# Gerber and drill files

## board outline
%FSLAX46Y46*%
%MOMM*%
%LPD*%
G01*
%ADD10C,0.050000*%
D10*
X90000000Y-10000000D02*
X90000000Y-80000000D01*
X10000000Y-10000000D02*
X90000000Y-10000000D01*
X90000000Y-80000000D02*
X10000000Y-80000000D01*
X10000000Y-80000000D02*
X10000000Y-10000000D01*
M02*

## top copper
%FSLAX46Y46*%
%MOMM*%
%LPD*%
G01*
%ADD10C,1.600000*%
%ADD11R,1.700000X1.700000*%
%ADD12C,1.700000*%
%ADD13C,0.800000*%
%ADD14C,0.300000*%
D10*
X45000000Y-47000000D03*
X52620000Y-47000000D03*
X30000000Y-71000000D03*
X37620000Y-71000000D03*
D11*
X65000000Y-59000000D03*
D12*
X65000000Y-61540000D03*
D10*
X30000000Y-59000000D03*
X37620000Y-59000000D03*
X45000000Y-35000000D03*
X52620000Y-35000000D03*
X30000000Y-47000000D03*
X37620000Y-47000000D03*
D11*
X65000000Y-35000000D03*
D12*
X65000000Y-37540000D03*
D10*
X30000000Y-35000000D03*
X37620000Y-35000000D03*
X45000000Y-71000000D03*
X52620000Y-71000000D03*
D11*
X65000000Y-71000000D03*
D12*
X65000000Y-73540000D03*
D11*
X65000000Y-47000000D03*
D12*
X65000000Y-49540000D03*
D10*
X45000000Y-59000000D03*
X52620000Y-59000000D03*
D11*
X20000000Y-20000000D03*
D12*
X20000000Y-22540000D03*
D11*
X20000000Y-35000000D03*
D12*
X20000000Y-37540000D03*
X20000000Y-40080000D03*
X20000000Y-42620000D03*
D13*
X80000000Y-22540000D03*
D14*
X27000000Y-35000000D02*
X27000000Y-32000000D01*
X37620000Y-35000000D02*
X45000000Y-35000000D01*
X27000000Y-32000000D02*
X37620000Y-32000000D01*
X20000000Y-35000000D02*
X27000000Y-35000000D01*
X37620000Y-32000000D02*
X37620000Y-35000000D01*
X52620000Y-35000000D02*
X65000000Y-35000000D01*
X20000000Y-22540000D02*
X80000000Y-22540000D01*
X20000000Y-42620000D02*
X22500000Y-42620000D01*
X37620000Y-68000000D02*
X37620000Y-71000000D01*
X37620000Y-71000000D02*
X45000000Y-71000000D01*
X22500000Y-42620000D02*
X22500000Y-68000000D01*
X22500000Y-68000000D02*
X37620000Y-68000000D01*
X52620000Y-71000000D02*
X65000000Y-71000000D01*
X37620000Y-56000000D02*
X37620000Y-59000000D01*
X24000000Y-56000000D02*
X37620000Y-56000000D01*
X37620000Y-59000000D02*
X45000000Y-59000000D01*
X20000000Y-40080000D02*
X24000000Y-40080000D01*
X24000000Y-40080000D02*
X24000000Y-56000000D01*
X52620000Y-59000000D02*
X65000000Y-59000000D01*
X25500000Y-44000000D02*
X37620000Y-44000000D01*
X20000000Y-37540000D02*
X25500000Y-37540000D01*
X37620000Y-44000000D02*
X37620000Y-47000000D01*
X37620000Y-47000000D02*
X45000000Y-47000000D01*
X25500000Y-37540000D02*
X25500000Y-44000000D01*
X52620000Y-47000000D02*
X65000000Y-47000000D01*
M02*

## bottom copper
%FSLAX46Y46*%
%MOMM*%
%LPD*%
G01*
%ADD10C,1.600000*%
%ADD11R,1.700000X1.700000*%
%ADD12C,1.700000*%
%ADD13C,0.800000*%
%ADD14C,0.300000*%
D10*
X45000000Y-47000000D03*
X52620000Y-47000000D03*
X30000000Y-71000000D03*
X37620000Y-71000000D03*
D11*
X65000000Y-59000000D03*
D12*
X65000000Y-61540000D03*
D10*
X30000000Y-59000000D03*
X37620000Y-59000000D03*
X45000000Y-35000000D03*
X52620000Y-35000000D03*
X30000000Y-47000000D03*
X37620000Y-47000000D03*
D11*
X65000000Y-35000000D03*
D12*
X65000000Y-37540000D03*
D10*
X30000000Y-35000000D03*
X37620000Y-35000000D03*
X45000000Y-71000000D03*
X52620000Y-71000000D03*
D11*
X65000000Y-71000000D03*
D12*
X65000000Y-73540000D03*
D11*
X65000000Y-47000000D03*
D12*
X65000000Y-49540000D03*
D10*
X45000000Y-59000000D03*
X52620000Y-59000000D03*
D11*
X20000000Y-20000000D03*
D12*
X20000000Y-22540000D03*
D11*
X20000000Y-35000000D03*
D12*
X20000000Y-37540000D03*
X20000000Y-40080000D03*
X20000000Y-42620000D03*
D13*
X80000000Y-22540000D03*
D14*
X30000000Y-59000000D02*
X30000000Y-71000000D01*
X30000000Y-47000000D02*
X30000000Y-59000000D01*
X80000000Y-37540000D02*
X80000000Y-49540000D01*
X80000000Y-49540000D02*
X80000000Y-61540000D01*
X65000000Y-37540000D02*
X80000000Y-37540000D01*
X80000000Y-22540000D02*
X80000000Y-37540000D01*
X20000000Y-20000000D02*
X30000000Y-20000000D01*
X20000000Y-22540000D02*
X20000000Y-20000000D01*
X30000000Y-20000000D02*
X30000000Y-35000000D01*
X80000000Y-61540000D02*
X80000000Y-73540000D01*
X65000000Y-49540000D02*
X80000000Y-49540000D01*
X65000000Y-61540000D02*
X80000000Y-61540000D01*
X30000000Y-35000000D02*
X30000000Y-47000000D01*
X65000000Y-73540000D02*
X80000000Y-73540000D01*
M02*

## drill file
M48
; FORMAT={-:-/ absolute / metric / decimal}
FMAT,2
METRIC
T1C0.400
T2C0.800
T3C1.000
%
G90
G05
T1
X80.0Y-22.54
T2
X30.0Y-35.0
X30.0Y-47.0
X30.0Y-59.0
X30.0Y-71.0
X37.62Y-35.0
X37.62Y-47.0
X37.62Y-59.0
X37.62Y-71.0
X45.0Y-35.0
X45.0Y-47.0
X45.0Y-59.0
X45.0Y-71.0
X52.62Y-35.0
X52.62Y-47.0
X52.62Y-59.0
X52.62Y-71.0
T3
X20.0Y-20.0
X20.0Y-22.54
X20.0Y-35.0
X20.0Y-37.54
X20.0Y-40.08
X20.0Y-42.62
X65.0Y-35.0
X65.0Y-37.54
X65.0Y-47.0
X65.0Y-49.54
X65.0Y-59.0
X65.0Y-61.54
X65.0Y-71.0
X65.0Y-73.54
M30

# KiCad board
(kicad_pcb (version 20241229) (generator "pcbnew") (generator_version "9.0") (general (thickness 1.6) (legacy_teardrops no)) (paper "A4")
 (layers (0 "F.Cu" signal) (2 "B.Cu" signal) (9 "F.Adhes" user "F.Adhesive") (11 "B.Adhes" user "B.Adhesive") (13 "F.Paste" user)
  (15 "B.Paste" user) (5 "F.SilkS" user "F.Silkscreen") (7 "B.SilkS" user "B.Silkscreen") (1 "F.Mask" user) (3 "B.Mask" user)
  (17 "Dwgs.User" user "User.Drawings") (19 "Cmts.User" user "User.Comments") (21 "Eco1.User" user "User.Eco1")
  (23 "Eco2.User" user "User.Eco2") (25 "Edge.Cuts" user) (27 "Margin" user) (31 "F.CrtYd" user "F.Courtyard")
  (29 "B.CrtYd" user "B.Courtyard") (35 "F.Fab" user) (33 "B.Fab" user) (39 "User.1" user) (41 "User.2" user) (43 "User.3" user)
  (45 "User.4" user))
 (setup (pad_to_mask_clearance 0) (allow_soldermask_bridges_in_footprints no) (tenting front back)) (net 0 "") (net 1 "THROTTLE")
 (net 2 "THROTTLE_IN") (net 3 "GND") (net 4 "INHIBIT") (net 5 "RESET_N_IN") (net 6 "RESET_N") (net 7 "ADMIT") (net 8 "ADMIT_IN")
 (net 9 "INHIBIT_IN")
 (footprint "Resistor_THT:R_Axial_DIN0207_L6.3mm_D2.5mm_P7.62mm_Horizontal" (layer "F.Cu") (at 45 47)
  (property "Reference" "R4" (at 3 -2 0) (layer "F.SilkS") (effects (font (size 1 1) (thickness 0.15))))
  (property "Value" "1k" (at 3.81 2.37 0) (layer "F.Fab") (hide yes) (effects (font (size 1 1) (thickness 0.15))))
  (pad "1" thru_hole circle (at 0 0) (size 1.6 1.6) (drill 0.8) (layers "*.Cu" "*.Mask") (remove_unused_layers no) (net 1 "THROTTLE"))
  (pad "2" thru_hole circle (at 7.62 0) (size 1.6 1.6) (drill 0.8) (layers "*.Cu" "*.Mask") (remove_unused_layers no) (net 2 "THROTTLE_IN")))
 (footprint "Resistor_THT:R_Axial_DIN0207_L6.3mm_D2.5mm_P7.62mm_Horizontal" (layer "F.Cu") (at 30 71)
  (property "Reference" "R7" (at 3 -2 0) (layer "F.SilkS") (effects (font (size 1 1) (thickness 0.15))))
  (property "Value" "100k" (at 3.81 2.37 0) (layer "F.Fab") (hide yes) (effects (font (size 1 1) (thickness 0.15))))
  (pad "1" thru_hole circle (at 0 0) (size 1.6 1.6) (drill 0.8) (layers "*.Cu" "*.Mask") (remove_unused_layers no) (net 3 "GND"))
  (pad "2" thru_hole circle (at 7.62 0) (size 1.6 1.6) (drill 0.8) (layers "*.Cu" "*.Mask") (remove_unused_layers no) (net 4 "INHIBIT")))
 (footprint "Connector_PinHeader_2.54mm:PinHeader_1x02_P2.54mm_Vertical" (layer "F.Cu") (at 65 59)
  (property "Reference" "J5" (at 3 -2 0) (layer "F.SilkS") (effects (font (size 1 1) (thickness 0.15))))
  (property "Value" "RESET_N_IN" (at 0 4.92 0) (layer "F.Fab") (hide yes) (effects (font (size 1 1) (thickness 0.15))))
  (pad "1" thru_hole rect (at 0 0) (size 1.7 1.7) (drill 1) (layers "*.Cu" "*.Mask") (remove_unused_layers no) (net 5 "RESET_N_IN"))
  (pad "2" thru_hole circle (at 0 2.54) (size 1.7 1.7) (drill 1) (layers "*.Cu" "*.Mask") (remove_unused_layers no) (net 3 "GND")))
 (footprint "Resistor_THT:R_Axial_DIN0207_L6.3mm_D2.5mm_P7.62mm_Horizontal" (layer "F.Cu") (at 30 59)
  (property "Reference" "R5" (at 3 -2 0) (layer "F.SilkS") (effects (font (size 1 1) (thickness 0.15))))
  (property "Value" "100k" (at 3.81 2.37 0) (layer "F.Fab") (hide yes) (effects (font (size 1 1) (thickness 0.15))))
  (pad "1" thru_hole circle (at 0 0) (size 1.6 1.6) (drill 0.8) (layers "*.Cu" "*.Mask") (remove_unused_layers no) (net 3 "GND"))
  (pad "2" thru_hole circle (at 7.62 0) (size 1.6 1.6) (drill 0.8) (layers "*.Cu" "*.Mask") (remove_unused_layers no) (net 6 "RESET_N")))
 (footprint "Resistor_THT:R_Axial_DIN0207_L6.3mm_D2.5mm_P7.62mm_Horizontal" (layer "F.Cu") (at 45 35)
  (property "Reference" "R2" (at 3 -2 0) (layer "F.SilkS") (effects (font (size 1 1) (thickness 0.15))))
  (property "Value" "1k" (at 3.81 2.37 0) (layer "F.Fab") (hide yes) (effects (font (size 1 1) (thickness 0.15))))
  (pad "1" thru_hole circle (at 0 0) (size 1.6 1.6) (drill 0.8) (layers "*.Cu" "*.Mask") (remove_unused_layers no) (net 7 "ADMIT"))
  (pad "2" thru_hole circle (at 7.62 0) (size 1.6 1.6) (drill 0.8) (layers "*.Cu" "*.Mask") (remove_unused_layers no) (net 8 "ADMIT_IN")))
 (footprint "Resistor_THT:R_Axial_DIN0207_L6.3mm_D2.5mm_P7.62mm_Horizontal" (layer "F.Cu") (at 30 47)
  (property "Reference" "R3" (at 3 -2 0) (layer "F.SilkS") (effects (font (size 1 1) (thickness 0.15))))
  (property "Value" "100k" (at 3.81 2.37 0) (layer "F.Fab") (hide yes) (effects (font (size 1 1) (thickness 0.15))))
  (pad "1" thru_hole circle (at 0 0) (size 1.6 1.6) (drill 0.8) (layers "*.Cu" "*.Mask") (remove_unused_layers no) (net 3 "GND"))
  (pad "2" thru_hole circle (at 7.62 0) (size 1.6 1.6) (drill 0.8) (layers "*.Cu" "*.Mask") (remove_unused_layers no) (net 1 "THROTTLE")))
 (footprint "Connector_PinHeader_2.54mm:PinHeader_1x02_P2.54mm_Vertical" (layer "F.Cu") (at 65 35)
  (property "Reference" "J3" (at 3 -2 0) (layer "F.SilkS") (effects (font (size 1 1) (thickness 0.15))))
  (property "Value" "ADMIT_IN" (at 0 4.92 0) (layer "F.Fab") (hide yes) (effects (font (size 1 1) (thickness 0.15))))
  (pad "1" thru_hole rect (at 0 0) (size 1.7 1.7) (drill 1) (layers "*.Cu" "*.Mask") (remove_unused_layers no) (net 8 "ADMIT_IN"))
  (pad "2" thru_hole circle (at 0 2.54) (size 1.7 1.7) (drill 1) (layers "*.Cu" "*.Mask") (remove_unused_layers no) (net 3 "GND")))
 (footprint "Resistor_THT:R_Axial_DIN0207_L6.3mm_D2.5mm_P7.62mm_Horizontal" (layer "F.Cu") (at 30 35)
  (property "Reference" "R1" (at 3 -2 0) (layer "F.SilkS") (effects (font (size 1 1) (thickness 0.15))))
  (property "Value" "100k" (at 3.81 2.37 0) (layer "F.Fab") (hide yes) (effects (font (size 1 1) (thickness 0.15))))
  (pad "1" thru_hole circle (at 0 0) (size 1.6 1.6) (drill 0.8) (layers "*.Cu" "*.Mask") (remove_unused_layers no) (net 3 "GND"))
  (pad "2" thru_hole circle (at 7.62 0) (size 1.6 1.6) (drill 0.8) (layers "*.Cu" "*.Mask") (remove_unused_layers no) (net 7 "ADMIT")))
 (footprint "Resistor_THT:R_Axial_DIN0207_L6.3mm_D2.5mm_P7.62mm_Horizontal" (layer "F.Cu") (at 45 71)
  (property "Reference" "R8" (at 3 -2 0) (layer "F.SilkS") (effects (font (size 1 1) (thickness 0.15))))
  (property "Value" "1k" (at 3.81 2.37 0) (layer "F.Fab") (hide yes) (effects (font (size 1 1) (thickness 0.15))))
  (pad "1" thru_hole circle (at 0 0) (size 1.6 1.6) (drill 0.8) (layers "*.Cu" "*.Mask") (remove_unused_layers no) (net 4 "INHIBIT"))
  (pad "2" thru_hole circle (at 7.62 0) (size 1.6 1.6) (drill 0.8) (layers "*.Cu" "*.Mask") (remove_unused_layers no) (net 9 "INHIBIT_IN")))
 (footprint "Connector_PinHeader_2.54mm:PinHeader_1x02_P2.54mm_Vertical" (layer "F.Cu") (at 65 71)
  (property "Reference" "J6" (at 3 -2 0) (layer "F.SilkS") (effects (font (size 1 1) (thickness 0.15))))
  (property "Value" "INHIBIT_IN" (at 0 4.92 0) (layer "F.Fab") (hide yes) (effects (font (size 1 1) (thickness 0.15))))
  (pad "1" thru_hole rect (at 0 0) (size 1.7 1.7) (drill 1) (layers "*.Cu" "*.Mask") (remove_unused_layers no) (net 9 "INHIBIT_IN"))
  (pad "2" thru_hole circle (at 0 2.54) (size 1.7 1.7) (drill 1) (layers "*.Cu" "*.Mask") (remove_unused_layers no) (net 3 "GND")))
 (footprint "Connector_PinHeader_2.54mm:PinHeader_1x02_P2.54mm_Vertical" (layer "F.Cu") (at 65 47)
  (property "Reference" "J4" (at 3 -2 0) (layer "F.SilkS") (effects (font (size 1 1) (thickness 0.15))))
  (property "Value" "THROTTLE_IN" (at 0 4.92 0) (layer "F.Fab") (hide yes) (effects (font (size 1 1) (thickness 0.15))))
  (pad "1" thru_hole rect (at 0 0) (size 1.7 1.7) (drill 1) (layers "*.Cu" "*.Mask") (remove_unused_layers no) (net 2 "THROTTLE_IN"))
  (pad "2" thru_hole circle (at 0 2.54) (size 1.7 1.7) (drill 1) (layers "*.Cu" "*.Mask") (remove_unused_layers no) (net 3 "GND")))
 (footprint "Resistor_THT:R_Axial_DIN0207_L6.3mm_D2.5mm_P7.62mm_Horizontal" (layer "F.Cu") (at 45 59)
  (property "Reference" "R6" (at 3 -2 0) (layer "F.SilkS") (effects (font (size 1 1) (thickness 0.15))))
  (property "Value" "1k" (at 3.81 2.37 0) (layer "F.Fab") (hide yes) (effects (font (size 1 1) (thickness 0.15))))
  (pad "1" thru_hole circle (at 0 0) (size 1.6 1.6) (drill 0.8) (layers "*.Cu" "*.Mask") (remove_unused_layers no) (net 6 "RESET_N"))
  (pad "2" thru_hole circle (at 7.62 0) (size 1.6 1.6) (drill 0.8) (layers "*.Cu" "*.Mask") (remove_unused_layers no) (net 5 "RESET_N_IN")))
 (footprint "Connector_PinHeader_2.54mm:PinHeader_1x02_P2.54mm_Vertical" (layer "F.Cu") (at 20 20)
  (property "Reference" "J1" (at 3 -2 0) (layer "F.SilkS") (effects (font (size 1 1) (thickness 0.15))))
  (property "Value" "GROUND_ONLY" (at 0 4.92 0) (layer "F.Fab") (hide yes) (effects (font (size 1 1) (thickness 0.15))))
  (pad "1" thru_hole rect (at 0 0) (size 1.7 1.7) (drill 1) (layers "*.Cu" "*.Mask") (remove_unused_layers no) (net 3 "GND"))
  (pad "2" thru_hole circle (at 0 2.54) (size 1.7 1.7) (drill 1) (layers "*.Cu" "*.Mask") (remove_unused_layers no) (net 3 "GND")))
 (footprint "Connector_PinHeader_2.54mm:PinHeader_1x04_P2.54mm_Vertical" (layer "F.Cu") (at 20 35)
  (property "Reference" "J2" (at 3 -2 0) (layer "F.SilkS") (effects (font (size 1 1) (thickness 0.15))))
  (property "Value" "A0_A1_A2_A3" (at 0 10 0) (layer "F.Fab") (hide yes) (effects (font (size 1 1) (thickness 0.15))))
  (pad "1" thru_hole rect (at 0 0) (size 1.7 1.7) (drill 1) (layers "*.Cu" "*.Mask") (remove_unused_layers no) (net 7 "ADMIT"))
  (pad "2" thru_hole circle (at 0 2.54) (size 1.7 1.7) (drill 1) (layers "*.Cu" "*.Mask") (remove_unused_layers no) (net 1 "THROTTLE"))
  (pad "3" thru_hole circle (at 0 5.08) (size 1.7 1.7) (drill 1) (layers "*.Cu" "*.Mask") (remove_unused_layers no) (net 6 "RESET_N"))
  (pad "4" thru_hole circle (at 0 7.62) (size 1.7 1.7) (drill 1) (layers "*.Cu" "*.Mask") (remove_unused_layers no) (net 4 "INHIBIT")))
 (gr_line (start 90 10) (end 90 80) (stroke (width 0.05) (type default)) (layer "Edge.Cuts"))
 (gr_line (start 10 10) (end 90 10) (stroke (width 0.05) (type default)) (layer "Edge.Cuts"))
 (gr_line (start 90 80) (end 10 80) (stroke (width 0.05) (type default)) (layer "Edge.Cuts"))
 (gr_line (start 10 80) (end 10 10) (stroke (width 0.05) (type default)) (layer "Edge.Cuts"))
 (segment (start 27 35) (end 27 32) (width 0.3) (layer "F.Cu") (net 7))
 (segment (start 37.62 35) (end 45 35) (width 0.3) (layer "F.Cu") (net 7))
 (segment (start 27 32) (end 37.62 32) (width 0.3) (layer "F.Cu") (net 7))
 (segment (start 20 35) (end 27 35) (width 0.3) (layer "F.Cu") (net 7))
 (segment (start 37.62 32) (end 37.62 35) (width 0.3) (layer "F.Cu") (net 7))
 (segment (start 52.62 35) (end 65 35) (width 0.3) (layer "F.Cu") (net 8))
 (segment (start 20 22.54) (end 80 22.54) (width 0.3) (layer "F.Cu") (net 3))
 (via (at 80 22.54) (size 0.8) (drill 0.4) (layers "F.Cu" "B.Cu") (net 3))
 (segment (start 30 59) (end 30 71) (width 0.3) (layer "B.Cu") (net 3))
 (segment (start 30 47) (end 30 59) (width 0.3) (layer "B.Cu") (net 3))
 (segment (start 80 37.54) (end 80 49.54) (width 0.3) (layer "B.Cu") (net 3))
 (segment (start 80 49.54) (end 80 61.54) (width 0.3) (layer "B.Cu") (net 3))
 (segment (start 65 37.54) (end 80 37.54) (width 0.3) (layer "B.Cu") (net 3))
 (segment (start 80 22.54) (end 80 37.54) (width 0.3) (layer "B.Cu") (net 3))
 (segment (start 20 20) (end 30 20) (width 0.3) (layer "B.Cu") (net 3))
 (segment (start 20 22.54) (end 20 20) (width 0.3) (layer "B.Cu") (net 3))
 (segment (start 30 20) (end 30 35) (width 0.3) (layer "B.Cu") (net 3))
 (segment (start 80 61.54) (end 80 73.54) (width 0.3) (layer "B.Cu") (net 3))
 (segment (start 65 49.54) (end 80 49.54) (width 0.3) (layer "B.Cu") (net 3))
 (segment (start 65 61.54) (end 80 61.54) (width 0.3) (layer "B.Cu") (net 3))
 (segment (start 30 35) (end 30 47) (width 0.3) (layer "B.Cu") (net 3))
 (segment (start 65 73.54) (end 80 73.54) (width 0.3) (layer "B.Cu") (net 3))
 (segment (start 20 42.62) (end 22.5 42.62) (width 0.3) (layer "F.Cu") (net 4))
 (segment (start 37.62 68) (end 37.62 71) (width 0.3) (layer "F.Cu") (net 4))
 (segment (start 37.62 71) (end 45 71) (width 0.3) (layer "F.Cu") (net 4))
 (segment (start 22.5 42.62) (end 22.5 68) (width 0.3) (layer "F.Cu") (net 4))
 (segment (start 22.5 68) (end 37.62 68) (width 0.3) (layer "F.Cu") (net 4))
 (segment (start 52.62 71) (end 65 71) (width 0.3) (layer "F.Cu") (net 9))
 (segment (start 37.62 56) (end 37.62 59) (width 0.3) (layer "F.Cu") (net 6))
 (segment (start 24 56) (end 37.62 56) (width 0.3) (layer "F.Cu") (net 6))
 (segment (start 37.62 59) (end 45 59) (width 0.3) (layer "F.Cu") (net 6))
 (segment (start 20 40.08) (end 24 40.08) (width 0.3) (layer "F.Cu") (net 6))
 (segment (start 24 40.08) (end 24 56) (width 0.3) (layer "F.Cu") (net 6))
 (segment (start 52.62 59) (end 65 59) (width 0.3) (layer "F.Cu") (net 5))
 (segment (start 25.5 44) (end 37.62 44) (width 0.3) (layer "F.Cu") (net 1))
 (segment (start 20 37.54) (end 25.5 37.54) (width 0.3) (layer "F.Cu") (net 1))
 (segment (start 37.62 44) (end 37.62 47) (width 0.3) (layer "F.Cu") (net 1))
 (segment (start 37.62 47) (end 45 47) (width 0.3) (layer "F.Cu") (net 1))
 (segment (start 25.5 37.54) (end 25.5 44) (width 0.3) (layer "F.Cu") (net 1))
 (segment (start 52.62 47) (end 65 47) (width 0.3) (layer "F.Cu") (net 2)))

